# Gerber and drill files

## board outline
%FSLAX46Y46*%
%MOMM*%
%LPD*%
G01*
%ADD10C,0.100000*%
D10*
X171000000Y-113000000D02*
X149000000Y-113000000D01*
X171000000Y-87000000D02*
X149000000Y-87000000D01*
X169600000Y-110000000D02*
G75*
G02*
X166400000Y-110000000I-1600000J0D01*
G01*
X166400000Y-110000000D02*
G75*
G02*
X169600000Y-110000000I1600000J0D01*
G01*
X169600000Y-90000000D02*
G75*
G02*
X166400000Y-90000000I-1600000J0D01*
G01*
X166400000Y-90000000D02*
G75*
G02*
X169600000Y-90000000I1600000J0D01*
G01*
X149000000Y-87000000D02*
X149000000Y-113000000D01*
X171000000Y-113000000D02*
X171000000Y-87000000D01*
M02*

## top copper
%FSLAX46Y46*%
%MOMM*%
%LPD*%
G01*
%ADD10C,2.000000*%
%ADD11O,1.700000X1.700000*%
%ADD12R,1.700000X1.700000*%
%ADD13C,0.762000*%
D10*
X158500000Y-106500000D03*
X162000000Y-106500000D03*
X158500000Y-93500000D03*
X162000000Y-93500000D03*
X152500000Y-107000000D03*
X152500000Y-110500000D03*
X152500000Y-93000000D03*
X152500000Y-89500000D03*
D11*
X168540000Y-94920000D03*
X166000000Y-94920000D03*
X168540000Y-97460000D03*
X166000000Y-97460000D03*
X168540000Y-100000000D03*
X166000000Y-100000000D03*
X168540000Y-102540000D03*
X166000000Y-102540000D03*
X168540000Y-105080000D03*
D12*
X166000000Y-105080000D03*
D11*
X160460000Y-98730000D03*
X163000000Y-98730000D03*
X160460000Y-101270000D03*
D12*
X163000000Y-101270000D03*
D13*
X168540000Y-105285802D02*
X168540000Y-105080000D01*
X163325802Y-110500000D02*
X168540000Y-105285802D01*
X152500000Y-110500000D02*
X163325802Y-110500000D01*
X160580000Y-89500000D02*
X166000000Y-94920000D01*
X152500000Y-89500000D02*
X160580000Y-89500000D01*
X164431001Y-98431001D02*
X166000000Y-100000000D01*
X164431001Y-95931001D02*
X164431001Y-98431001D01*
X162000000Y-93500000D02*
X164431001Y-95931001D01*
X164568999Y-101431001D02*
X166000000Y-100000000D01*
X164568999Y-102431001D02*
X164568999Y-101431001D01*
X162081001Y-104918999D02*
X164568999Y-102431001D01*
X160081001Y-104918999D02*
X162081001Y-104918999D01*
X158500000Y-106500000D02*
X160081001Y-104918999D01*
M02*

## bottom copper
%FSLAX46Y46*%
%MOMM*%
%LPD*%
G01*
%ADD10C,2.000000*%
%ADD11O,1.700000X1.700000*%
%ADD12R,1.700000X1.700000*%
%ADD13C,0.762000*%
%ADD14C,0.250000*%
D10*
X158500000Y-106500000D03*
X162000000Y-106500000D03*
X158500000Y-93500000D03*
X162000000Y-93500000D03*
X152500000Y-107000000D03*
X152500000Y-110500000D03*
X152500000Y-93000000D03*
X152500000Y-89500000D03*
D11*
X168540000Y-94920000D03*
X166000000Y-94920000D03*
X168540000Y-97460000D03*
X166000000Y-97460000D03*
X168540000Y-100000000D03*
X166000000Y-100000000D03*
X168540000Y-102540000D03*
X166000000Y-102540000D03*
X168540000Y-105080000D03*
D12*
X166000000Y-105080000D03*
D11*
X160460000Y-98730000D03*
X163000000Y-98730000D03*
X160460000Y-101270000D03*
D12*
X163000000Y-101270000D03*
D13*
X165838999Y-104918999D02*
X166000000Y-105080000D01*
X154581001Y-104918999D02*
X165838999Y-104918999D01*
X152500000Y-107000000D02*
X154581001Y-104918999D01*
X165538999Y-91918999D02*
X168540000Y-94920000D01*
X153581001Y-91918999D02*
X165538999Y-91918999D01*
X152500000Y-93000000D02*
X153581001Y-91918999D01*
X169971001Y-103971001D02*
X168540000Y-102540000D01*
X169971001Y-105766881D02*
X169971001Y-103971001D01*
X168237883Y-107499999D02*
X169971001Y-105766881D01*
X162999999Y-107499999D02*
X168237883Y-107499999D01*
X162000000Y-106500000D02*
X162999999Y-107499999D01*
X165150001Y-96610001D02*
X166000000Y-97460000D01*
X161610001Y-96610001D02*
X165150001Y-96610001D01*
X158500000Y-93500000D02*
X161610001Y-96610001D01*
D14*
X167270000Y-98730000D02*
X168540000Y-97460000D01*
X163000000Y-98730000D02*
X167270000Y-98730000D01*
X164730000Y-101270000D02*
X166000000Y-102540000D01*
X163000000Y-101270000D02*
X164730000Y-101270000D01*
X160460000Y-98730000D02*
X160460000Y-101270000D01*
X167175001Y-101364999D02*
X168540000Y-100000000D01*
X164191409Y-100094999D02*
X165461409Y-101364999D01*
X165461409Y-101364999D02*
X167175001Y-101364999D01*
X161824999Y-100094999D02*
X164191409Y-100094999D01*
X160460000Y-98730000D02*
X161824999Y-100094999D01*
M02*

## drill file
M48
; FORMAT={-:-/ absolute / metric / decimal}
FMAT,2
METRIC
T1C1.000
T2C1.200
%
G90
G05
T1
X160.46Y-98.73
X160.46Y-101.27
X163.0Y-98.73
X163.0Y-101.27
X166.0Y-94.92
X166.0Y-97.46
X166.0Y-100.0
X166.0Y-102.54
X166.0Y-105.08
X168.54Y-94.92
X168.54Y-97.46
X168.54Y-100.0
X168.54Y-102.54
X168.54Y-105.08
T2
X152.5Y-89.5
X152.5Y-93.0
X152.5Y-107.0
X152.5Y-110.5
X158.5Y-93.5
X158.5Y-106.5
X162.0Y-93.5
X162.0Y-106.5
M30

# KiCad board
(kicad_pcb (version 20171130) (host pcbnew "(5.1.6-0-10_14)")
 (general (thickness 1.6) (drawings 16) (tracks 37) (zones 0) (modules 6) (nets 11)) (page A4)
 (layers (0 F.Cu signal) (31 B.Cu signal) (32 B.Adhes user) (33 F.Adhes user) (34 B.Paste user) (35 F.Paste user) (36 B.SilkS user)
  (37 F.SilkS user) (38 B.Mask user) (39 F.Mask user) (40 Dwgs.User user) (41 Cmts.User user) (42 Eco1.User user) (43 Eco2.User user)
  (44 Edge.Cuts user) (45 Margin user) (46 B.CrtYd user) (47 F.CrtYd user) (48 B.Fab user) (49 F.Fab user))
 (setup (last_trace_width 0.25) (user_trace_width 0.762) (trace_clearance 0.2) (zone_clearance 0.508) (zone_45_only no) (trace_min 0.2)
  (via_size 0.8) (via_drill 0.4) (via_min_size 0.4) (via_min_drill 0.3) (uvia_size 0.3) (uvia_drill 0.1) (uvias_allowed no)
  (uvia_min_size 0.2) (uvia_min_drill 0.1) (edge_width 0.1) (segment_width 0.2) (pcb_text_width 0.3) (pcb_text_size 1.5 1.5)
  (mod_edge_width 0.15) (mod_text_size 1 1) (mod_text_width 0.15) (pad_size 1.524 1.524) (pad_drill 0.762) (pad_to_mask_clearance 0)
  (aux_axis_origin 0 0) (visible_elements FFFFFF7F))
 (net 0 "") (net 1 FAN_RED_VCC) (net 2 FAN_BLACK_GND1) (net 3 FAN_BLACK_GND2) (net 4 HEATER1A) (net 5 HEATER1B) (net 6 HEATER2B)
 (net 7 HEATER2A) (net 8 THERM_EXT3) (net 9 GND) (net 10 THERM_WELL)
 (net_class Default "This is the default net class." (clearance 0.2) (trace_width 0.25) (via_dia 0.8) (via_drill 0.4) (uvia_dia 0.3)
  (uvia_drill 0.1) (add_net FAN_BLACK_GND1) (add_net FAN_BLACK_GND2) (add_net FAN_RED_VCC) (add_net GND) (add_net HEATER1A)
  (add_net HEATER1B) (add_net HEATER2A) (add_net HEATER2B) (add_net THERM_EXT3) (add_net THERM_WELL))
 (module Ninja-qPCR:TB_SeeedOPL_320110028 (layer F.Cu) (at 158.5 106.5)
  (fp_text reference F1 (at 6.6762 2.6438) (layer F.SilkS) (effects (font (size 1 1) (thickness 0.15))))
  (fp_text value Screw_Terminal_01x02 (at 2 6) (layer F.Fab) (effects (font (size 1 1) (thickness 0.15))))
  (pad 1 thru_hole circle (at 0 0) (size 2 2) (drill 1.2) (layers *.Cu *.Mask) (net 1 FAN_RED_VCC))
  (pad 2 thru_hole circle (at 3.5 0) (size 2 2) (drill 1.2) (layers *.Cu *.Mask) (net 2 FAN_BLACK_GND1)))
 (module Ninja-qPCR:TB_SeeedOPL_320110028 (layer F.Cu) (at 162 93.5 180)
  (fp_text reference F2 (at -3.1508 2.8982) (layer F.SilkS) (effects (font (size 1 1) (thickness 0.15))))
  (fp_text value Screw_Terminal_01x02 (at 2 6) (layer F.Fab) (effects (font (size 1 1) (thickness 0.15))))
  (pad 2 thru_hole circle (at 3.5 0 180) (size 2 2) (drill 1.2) (layers *.Cu *.Mask) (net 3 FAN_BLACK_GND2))
  (pad 1 thru_hole circle (at 0 0 180) (size 2 2) (drill 1.2) (layers *.Cu *.Mask) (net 1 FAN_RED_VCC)))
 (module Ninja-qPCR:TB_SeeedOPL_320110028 (layer F.Cu) (at 152.5 107 270)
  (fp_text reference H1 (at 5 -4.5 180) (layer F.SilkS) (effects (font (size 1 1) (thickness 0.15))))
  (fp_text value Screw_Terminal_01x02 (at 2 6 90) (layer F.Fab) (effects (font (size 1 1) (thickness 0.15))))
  (pad 1 thru_hole circle (at 0 0 270) (size 2 2) (drill 1.2) (layers *.Cu *.Mask) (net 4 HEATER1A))
  (pad 2 thru_hole circle (at 3.5 0 270) (size 2 2) (drill 1.2) (layers *.Cu *.Mask) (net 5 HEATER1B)))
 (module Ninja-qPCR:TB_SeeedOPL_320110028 (layer F.Cu) (at 152.5 89.5 270)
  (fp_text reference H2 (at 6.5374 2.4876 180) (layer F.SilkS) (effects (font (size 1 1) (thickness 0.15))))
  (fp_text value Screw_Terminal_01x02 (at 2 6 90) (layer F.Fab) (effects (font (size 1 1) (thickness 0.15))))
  (pad 2 thru_hole circle (at 3.5 0 270) (size 2 2) (drill 1.2) (layers *.Cu *.Mask) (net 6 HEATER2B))
  (pad 1 thru_hole circle (at 0 0 270) (size 2 2) (drill 1.2) (layers *.Cu *.Mask) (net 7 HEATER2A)))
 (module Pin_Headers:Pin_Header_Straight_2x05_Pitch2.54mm (layer B.Cu) (at 166 105.08)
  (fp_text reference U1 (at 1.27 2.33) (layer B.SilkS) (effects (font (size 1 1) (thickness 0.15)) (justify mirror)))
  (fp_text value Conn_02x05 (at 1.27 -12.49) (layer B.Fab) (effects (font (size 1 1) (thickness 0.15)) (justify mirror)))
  (pad 10 thru_hole oval (at 2.54 -10.16) (size 1.7 1.7) (drill 1) (layers *.Cu *.Mask) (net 6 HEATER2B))
  (pad 9 thru_hole oval (at 0 -10.16) (size 1.7 1.7) (drill 1) (layers *.Cu *.Mask) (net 7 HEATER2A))
  (pad 8 thru_hole oval (at 2.54 -7.62) (size 1.7 1.7) (drill 1) (layers *.Cu *.Mask) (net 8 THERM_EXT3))
  (pad 7 thru_hole oval (at 0 -7.62) (size 1.7 1.7) (drill 1) (layers *.Cu *.Mask) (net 3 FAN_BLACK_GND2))
  (pad 6 thru_hole oval (at 2.54 -5.08) (size 1.7 1.7) (drill 1) (layers *.Cu *.Mask) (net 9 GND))
  (pad 5 thru_hole oval (at 0 -5.08) (size 1.7 1.7) (drill 1) (layers *.Cu *.Mask) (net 1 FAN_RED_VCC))
  (pad 4 thru_hole oval (at 2.54 -2.54) (size 1.7 1.7) (drill 1) (layers *.Cu *.Mask) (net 2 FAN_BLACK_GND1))
  (pad 3 thru_hole oval (at 0 -2.54) (size 1.7 1.7) (drill 1) (layers *.Cu *.Mask) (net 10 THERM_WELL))
  (pad 2 thru_hole oval (at 2.54 0) (size 1.7 1.7) (drill 1) (layers *.Cu *.Mask) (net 5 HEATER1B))
  (pad 1 thru_hole rect (at 0 0) (size 1.7 1.7) (drill 1) (layers *.Cu *.Mask) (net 4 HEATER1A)))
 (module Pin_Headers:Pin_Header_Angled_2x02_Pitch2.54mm (layer F.Cu) (at 163 101.27 180)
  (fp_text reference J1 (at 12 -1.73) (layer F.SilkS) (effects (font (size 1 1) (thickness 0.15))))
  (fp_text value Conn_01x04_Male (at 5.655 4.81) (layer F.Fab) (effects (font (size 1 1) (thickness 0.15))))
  (pad 4 thru_hole oval (at 2.54 2.54 180) (size 1.7 1.7) (drill 1) (layers *.Cu *.Mask) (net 9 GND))
  (pad 3 thru_hole oval (at 0 2.54 180) (size 1.7 1.7) (drill 1) (layers *.Cu *.Mask) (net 8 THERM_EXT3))
  (pad 2 thru_hole oval (at 2.54 0 180) (size 1.7 1.7) (drill 1) (layers *.Cu *.Mask) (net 9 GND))
  (pad 1 thru_hole rect (at 0 0 180) (size 1.7 1.7) (drill 1) (layers *.Cu *.Mask) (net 10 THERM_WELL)))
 (gr_line (start 171 113) (end 149 113) (layer Edge.Cuts) (width 0.1))
 (gr_line (start 171 87) (end 149 87) (layer Edge.Cuts) (width 0.1))
 (gr_circle (center 168 110) (end 169.6 110) (layer Edge.Cuts) (width 0.1))
 (gr_circle (center 168 90) (end 169.6 90) (layer Edge.Cuts) (width 0.1))
 (gr_line (start 149 87) (end 149 113) (layer Edge.Cuts) (width 0.1))
 (gr_line (start 171 113) (end 171 87) (layer Edge.Cuts) (width 0.1))
 (segment (start 165.838999 104.918999) (end 166 105.08) (width 0.762) (layer B.Cu) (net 4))
 (segment (start 154.581001 104.918999) (end 165.838999 104.918999) (width 0.762) (layer B.Cu) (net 4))
 (segment (start 152.5 107) (end 154.581001 104.918999) (width 0.762) (layer B.Cu) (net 4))
 (segment (start 168.54 105.285802) (end 168.54 105.08) (width 0.762) (layer F.Cu) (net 5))
 (segment (start 163.325802 110.5) (end 168.54 105.285802) (width 0.762) (layer F.Cu) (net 5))
 (segment (start 152.5 110.5) (end 163.325802 110.5) (width 0.762) (layer F.Cu) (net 5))
 (segment (start 165.538999 91.918999) (end 168.54 94.92) (width 0.762) (layer B.Cu) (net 6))
 (segment (start 153.581001 91.918999) (end 165.538999 91.918999) (width 0.762) (layer B.Cu) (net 6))
 (segment (start 152.5 93) (end 153.581001 91.918999) (width 0.762) (layer B.Cu) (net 6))
 (segment (start 160.58 89.5) (end 166 94.92) (width 0.762) (layer F.Cu) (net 7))
 (segment (start 152.5 89.5) (end 160.58 89.5) (width 0.762) (layer F.Cu) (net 7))
 (segment (start 164.431001 98.431001) (end 166 100) (width 0.762) (layer F.Cu) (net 1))
 (segment (start 164.431001 95.931001) (end 164.431001 98.431001) (width 0.762) (layer F.Cu) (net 1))
 (segment (start 162 93.5) (end 164.431001 95.931001) (width 0.762) (layer F.Cu) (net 1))
 (segment (start 164.568999 101.431001) (end 166 100) (width 0.762) (layer F.Cu) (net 1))
 (segment (start 164.568999 102.431001) (end 164.568999 101.431001) (width 0.762) (layer F.Cu) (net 1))
 (segment (start 162.081001 104.918999) (end 164.568999 102.431001) (width 0.762) (layer F.Cu) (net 1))
 (segment (start 160.081001 104.918999) (end 162.081001 104.918999) (width 0.762) (layer F.Cu) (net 1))
 (segment (start 158.5 106.5) (end 160.081001 104.918999) (width 0.762) (layer F.Cu) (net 1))
 (segment (start 169.971001 103.971001) (end 168.54 102.54) (width 0.762) (layer B.Cu) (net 2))
 (segment (start 169.971001 105.766881) (end 169.971001 103.971001) (width 0.762) (layer B.Cu) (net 2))
 (segment (start 168.237883 107.499999) (end 169.971001 105.766881) (width 0.762) (layer B.Cu) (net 2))
 (segment (start 162.999999 107.499999) (end 168.237883 107.499999) (width 0.762) (layer B.Cu) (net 2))
 (segment (start 162 106.5) (end 162.999999 107.499999) (width 0.762) (layer B.Cu) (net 2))
 (segment (start 165.150001 96.610001) (end 166 97.46) (width 0.762) (layer B.Cu) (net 3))
 (segment (start 161.610001 96.610001) (end 165.150001 96.610001) (width 0.762) (layer B.Cu) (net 3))
 (segment (start 158.5 93.5) (end 161.610001 96.610001) (width 0.762) (layer B.Cu) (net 3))
 (segment (start 167.27 98.73) (end 168.54 97.46) (width 0.25) (layer B.Cu) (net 8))
 (segment (start 163 98.73) (end 167.27 98.73) (width 0.25) (layer B.Cu) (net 8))
 (segment (start 164.73 101.27) (end 166 102.54) (width 0.25) (layer B.Cu) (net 10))
 (segment (start 163 101.27) (end 164.73 101.27) (width 0.25) (layer B.Cu) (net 10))
 (segment (start 160.46 98.73) (end 160.46 101.27) (width 0.25) (layer B.Cu) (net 9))
 (segment (start 167.175001 101.364999) (end 168.54 100) (width 0.25) (layer B.Cu) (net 9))
 (segment (start 164.191409 100.094999) (end 165.461409 101.364999) (width 0.25) (layer B.Cu) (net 9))
 (segment (start 165.461409 101.364999) (end 167.175001 101.364999) (width 0.25) (layer B.Cu) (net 9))
 (segment (start 161.824999 100.094999) (end 164.191409 100.094999) (width 0.25) (layer B.Cu) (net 9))
 (segment (start 160.46 98.73) (end 161.824999 100.094999) (width 0.25) (layer B.Cu) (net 9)))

